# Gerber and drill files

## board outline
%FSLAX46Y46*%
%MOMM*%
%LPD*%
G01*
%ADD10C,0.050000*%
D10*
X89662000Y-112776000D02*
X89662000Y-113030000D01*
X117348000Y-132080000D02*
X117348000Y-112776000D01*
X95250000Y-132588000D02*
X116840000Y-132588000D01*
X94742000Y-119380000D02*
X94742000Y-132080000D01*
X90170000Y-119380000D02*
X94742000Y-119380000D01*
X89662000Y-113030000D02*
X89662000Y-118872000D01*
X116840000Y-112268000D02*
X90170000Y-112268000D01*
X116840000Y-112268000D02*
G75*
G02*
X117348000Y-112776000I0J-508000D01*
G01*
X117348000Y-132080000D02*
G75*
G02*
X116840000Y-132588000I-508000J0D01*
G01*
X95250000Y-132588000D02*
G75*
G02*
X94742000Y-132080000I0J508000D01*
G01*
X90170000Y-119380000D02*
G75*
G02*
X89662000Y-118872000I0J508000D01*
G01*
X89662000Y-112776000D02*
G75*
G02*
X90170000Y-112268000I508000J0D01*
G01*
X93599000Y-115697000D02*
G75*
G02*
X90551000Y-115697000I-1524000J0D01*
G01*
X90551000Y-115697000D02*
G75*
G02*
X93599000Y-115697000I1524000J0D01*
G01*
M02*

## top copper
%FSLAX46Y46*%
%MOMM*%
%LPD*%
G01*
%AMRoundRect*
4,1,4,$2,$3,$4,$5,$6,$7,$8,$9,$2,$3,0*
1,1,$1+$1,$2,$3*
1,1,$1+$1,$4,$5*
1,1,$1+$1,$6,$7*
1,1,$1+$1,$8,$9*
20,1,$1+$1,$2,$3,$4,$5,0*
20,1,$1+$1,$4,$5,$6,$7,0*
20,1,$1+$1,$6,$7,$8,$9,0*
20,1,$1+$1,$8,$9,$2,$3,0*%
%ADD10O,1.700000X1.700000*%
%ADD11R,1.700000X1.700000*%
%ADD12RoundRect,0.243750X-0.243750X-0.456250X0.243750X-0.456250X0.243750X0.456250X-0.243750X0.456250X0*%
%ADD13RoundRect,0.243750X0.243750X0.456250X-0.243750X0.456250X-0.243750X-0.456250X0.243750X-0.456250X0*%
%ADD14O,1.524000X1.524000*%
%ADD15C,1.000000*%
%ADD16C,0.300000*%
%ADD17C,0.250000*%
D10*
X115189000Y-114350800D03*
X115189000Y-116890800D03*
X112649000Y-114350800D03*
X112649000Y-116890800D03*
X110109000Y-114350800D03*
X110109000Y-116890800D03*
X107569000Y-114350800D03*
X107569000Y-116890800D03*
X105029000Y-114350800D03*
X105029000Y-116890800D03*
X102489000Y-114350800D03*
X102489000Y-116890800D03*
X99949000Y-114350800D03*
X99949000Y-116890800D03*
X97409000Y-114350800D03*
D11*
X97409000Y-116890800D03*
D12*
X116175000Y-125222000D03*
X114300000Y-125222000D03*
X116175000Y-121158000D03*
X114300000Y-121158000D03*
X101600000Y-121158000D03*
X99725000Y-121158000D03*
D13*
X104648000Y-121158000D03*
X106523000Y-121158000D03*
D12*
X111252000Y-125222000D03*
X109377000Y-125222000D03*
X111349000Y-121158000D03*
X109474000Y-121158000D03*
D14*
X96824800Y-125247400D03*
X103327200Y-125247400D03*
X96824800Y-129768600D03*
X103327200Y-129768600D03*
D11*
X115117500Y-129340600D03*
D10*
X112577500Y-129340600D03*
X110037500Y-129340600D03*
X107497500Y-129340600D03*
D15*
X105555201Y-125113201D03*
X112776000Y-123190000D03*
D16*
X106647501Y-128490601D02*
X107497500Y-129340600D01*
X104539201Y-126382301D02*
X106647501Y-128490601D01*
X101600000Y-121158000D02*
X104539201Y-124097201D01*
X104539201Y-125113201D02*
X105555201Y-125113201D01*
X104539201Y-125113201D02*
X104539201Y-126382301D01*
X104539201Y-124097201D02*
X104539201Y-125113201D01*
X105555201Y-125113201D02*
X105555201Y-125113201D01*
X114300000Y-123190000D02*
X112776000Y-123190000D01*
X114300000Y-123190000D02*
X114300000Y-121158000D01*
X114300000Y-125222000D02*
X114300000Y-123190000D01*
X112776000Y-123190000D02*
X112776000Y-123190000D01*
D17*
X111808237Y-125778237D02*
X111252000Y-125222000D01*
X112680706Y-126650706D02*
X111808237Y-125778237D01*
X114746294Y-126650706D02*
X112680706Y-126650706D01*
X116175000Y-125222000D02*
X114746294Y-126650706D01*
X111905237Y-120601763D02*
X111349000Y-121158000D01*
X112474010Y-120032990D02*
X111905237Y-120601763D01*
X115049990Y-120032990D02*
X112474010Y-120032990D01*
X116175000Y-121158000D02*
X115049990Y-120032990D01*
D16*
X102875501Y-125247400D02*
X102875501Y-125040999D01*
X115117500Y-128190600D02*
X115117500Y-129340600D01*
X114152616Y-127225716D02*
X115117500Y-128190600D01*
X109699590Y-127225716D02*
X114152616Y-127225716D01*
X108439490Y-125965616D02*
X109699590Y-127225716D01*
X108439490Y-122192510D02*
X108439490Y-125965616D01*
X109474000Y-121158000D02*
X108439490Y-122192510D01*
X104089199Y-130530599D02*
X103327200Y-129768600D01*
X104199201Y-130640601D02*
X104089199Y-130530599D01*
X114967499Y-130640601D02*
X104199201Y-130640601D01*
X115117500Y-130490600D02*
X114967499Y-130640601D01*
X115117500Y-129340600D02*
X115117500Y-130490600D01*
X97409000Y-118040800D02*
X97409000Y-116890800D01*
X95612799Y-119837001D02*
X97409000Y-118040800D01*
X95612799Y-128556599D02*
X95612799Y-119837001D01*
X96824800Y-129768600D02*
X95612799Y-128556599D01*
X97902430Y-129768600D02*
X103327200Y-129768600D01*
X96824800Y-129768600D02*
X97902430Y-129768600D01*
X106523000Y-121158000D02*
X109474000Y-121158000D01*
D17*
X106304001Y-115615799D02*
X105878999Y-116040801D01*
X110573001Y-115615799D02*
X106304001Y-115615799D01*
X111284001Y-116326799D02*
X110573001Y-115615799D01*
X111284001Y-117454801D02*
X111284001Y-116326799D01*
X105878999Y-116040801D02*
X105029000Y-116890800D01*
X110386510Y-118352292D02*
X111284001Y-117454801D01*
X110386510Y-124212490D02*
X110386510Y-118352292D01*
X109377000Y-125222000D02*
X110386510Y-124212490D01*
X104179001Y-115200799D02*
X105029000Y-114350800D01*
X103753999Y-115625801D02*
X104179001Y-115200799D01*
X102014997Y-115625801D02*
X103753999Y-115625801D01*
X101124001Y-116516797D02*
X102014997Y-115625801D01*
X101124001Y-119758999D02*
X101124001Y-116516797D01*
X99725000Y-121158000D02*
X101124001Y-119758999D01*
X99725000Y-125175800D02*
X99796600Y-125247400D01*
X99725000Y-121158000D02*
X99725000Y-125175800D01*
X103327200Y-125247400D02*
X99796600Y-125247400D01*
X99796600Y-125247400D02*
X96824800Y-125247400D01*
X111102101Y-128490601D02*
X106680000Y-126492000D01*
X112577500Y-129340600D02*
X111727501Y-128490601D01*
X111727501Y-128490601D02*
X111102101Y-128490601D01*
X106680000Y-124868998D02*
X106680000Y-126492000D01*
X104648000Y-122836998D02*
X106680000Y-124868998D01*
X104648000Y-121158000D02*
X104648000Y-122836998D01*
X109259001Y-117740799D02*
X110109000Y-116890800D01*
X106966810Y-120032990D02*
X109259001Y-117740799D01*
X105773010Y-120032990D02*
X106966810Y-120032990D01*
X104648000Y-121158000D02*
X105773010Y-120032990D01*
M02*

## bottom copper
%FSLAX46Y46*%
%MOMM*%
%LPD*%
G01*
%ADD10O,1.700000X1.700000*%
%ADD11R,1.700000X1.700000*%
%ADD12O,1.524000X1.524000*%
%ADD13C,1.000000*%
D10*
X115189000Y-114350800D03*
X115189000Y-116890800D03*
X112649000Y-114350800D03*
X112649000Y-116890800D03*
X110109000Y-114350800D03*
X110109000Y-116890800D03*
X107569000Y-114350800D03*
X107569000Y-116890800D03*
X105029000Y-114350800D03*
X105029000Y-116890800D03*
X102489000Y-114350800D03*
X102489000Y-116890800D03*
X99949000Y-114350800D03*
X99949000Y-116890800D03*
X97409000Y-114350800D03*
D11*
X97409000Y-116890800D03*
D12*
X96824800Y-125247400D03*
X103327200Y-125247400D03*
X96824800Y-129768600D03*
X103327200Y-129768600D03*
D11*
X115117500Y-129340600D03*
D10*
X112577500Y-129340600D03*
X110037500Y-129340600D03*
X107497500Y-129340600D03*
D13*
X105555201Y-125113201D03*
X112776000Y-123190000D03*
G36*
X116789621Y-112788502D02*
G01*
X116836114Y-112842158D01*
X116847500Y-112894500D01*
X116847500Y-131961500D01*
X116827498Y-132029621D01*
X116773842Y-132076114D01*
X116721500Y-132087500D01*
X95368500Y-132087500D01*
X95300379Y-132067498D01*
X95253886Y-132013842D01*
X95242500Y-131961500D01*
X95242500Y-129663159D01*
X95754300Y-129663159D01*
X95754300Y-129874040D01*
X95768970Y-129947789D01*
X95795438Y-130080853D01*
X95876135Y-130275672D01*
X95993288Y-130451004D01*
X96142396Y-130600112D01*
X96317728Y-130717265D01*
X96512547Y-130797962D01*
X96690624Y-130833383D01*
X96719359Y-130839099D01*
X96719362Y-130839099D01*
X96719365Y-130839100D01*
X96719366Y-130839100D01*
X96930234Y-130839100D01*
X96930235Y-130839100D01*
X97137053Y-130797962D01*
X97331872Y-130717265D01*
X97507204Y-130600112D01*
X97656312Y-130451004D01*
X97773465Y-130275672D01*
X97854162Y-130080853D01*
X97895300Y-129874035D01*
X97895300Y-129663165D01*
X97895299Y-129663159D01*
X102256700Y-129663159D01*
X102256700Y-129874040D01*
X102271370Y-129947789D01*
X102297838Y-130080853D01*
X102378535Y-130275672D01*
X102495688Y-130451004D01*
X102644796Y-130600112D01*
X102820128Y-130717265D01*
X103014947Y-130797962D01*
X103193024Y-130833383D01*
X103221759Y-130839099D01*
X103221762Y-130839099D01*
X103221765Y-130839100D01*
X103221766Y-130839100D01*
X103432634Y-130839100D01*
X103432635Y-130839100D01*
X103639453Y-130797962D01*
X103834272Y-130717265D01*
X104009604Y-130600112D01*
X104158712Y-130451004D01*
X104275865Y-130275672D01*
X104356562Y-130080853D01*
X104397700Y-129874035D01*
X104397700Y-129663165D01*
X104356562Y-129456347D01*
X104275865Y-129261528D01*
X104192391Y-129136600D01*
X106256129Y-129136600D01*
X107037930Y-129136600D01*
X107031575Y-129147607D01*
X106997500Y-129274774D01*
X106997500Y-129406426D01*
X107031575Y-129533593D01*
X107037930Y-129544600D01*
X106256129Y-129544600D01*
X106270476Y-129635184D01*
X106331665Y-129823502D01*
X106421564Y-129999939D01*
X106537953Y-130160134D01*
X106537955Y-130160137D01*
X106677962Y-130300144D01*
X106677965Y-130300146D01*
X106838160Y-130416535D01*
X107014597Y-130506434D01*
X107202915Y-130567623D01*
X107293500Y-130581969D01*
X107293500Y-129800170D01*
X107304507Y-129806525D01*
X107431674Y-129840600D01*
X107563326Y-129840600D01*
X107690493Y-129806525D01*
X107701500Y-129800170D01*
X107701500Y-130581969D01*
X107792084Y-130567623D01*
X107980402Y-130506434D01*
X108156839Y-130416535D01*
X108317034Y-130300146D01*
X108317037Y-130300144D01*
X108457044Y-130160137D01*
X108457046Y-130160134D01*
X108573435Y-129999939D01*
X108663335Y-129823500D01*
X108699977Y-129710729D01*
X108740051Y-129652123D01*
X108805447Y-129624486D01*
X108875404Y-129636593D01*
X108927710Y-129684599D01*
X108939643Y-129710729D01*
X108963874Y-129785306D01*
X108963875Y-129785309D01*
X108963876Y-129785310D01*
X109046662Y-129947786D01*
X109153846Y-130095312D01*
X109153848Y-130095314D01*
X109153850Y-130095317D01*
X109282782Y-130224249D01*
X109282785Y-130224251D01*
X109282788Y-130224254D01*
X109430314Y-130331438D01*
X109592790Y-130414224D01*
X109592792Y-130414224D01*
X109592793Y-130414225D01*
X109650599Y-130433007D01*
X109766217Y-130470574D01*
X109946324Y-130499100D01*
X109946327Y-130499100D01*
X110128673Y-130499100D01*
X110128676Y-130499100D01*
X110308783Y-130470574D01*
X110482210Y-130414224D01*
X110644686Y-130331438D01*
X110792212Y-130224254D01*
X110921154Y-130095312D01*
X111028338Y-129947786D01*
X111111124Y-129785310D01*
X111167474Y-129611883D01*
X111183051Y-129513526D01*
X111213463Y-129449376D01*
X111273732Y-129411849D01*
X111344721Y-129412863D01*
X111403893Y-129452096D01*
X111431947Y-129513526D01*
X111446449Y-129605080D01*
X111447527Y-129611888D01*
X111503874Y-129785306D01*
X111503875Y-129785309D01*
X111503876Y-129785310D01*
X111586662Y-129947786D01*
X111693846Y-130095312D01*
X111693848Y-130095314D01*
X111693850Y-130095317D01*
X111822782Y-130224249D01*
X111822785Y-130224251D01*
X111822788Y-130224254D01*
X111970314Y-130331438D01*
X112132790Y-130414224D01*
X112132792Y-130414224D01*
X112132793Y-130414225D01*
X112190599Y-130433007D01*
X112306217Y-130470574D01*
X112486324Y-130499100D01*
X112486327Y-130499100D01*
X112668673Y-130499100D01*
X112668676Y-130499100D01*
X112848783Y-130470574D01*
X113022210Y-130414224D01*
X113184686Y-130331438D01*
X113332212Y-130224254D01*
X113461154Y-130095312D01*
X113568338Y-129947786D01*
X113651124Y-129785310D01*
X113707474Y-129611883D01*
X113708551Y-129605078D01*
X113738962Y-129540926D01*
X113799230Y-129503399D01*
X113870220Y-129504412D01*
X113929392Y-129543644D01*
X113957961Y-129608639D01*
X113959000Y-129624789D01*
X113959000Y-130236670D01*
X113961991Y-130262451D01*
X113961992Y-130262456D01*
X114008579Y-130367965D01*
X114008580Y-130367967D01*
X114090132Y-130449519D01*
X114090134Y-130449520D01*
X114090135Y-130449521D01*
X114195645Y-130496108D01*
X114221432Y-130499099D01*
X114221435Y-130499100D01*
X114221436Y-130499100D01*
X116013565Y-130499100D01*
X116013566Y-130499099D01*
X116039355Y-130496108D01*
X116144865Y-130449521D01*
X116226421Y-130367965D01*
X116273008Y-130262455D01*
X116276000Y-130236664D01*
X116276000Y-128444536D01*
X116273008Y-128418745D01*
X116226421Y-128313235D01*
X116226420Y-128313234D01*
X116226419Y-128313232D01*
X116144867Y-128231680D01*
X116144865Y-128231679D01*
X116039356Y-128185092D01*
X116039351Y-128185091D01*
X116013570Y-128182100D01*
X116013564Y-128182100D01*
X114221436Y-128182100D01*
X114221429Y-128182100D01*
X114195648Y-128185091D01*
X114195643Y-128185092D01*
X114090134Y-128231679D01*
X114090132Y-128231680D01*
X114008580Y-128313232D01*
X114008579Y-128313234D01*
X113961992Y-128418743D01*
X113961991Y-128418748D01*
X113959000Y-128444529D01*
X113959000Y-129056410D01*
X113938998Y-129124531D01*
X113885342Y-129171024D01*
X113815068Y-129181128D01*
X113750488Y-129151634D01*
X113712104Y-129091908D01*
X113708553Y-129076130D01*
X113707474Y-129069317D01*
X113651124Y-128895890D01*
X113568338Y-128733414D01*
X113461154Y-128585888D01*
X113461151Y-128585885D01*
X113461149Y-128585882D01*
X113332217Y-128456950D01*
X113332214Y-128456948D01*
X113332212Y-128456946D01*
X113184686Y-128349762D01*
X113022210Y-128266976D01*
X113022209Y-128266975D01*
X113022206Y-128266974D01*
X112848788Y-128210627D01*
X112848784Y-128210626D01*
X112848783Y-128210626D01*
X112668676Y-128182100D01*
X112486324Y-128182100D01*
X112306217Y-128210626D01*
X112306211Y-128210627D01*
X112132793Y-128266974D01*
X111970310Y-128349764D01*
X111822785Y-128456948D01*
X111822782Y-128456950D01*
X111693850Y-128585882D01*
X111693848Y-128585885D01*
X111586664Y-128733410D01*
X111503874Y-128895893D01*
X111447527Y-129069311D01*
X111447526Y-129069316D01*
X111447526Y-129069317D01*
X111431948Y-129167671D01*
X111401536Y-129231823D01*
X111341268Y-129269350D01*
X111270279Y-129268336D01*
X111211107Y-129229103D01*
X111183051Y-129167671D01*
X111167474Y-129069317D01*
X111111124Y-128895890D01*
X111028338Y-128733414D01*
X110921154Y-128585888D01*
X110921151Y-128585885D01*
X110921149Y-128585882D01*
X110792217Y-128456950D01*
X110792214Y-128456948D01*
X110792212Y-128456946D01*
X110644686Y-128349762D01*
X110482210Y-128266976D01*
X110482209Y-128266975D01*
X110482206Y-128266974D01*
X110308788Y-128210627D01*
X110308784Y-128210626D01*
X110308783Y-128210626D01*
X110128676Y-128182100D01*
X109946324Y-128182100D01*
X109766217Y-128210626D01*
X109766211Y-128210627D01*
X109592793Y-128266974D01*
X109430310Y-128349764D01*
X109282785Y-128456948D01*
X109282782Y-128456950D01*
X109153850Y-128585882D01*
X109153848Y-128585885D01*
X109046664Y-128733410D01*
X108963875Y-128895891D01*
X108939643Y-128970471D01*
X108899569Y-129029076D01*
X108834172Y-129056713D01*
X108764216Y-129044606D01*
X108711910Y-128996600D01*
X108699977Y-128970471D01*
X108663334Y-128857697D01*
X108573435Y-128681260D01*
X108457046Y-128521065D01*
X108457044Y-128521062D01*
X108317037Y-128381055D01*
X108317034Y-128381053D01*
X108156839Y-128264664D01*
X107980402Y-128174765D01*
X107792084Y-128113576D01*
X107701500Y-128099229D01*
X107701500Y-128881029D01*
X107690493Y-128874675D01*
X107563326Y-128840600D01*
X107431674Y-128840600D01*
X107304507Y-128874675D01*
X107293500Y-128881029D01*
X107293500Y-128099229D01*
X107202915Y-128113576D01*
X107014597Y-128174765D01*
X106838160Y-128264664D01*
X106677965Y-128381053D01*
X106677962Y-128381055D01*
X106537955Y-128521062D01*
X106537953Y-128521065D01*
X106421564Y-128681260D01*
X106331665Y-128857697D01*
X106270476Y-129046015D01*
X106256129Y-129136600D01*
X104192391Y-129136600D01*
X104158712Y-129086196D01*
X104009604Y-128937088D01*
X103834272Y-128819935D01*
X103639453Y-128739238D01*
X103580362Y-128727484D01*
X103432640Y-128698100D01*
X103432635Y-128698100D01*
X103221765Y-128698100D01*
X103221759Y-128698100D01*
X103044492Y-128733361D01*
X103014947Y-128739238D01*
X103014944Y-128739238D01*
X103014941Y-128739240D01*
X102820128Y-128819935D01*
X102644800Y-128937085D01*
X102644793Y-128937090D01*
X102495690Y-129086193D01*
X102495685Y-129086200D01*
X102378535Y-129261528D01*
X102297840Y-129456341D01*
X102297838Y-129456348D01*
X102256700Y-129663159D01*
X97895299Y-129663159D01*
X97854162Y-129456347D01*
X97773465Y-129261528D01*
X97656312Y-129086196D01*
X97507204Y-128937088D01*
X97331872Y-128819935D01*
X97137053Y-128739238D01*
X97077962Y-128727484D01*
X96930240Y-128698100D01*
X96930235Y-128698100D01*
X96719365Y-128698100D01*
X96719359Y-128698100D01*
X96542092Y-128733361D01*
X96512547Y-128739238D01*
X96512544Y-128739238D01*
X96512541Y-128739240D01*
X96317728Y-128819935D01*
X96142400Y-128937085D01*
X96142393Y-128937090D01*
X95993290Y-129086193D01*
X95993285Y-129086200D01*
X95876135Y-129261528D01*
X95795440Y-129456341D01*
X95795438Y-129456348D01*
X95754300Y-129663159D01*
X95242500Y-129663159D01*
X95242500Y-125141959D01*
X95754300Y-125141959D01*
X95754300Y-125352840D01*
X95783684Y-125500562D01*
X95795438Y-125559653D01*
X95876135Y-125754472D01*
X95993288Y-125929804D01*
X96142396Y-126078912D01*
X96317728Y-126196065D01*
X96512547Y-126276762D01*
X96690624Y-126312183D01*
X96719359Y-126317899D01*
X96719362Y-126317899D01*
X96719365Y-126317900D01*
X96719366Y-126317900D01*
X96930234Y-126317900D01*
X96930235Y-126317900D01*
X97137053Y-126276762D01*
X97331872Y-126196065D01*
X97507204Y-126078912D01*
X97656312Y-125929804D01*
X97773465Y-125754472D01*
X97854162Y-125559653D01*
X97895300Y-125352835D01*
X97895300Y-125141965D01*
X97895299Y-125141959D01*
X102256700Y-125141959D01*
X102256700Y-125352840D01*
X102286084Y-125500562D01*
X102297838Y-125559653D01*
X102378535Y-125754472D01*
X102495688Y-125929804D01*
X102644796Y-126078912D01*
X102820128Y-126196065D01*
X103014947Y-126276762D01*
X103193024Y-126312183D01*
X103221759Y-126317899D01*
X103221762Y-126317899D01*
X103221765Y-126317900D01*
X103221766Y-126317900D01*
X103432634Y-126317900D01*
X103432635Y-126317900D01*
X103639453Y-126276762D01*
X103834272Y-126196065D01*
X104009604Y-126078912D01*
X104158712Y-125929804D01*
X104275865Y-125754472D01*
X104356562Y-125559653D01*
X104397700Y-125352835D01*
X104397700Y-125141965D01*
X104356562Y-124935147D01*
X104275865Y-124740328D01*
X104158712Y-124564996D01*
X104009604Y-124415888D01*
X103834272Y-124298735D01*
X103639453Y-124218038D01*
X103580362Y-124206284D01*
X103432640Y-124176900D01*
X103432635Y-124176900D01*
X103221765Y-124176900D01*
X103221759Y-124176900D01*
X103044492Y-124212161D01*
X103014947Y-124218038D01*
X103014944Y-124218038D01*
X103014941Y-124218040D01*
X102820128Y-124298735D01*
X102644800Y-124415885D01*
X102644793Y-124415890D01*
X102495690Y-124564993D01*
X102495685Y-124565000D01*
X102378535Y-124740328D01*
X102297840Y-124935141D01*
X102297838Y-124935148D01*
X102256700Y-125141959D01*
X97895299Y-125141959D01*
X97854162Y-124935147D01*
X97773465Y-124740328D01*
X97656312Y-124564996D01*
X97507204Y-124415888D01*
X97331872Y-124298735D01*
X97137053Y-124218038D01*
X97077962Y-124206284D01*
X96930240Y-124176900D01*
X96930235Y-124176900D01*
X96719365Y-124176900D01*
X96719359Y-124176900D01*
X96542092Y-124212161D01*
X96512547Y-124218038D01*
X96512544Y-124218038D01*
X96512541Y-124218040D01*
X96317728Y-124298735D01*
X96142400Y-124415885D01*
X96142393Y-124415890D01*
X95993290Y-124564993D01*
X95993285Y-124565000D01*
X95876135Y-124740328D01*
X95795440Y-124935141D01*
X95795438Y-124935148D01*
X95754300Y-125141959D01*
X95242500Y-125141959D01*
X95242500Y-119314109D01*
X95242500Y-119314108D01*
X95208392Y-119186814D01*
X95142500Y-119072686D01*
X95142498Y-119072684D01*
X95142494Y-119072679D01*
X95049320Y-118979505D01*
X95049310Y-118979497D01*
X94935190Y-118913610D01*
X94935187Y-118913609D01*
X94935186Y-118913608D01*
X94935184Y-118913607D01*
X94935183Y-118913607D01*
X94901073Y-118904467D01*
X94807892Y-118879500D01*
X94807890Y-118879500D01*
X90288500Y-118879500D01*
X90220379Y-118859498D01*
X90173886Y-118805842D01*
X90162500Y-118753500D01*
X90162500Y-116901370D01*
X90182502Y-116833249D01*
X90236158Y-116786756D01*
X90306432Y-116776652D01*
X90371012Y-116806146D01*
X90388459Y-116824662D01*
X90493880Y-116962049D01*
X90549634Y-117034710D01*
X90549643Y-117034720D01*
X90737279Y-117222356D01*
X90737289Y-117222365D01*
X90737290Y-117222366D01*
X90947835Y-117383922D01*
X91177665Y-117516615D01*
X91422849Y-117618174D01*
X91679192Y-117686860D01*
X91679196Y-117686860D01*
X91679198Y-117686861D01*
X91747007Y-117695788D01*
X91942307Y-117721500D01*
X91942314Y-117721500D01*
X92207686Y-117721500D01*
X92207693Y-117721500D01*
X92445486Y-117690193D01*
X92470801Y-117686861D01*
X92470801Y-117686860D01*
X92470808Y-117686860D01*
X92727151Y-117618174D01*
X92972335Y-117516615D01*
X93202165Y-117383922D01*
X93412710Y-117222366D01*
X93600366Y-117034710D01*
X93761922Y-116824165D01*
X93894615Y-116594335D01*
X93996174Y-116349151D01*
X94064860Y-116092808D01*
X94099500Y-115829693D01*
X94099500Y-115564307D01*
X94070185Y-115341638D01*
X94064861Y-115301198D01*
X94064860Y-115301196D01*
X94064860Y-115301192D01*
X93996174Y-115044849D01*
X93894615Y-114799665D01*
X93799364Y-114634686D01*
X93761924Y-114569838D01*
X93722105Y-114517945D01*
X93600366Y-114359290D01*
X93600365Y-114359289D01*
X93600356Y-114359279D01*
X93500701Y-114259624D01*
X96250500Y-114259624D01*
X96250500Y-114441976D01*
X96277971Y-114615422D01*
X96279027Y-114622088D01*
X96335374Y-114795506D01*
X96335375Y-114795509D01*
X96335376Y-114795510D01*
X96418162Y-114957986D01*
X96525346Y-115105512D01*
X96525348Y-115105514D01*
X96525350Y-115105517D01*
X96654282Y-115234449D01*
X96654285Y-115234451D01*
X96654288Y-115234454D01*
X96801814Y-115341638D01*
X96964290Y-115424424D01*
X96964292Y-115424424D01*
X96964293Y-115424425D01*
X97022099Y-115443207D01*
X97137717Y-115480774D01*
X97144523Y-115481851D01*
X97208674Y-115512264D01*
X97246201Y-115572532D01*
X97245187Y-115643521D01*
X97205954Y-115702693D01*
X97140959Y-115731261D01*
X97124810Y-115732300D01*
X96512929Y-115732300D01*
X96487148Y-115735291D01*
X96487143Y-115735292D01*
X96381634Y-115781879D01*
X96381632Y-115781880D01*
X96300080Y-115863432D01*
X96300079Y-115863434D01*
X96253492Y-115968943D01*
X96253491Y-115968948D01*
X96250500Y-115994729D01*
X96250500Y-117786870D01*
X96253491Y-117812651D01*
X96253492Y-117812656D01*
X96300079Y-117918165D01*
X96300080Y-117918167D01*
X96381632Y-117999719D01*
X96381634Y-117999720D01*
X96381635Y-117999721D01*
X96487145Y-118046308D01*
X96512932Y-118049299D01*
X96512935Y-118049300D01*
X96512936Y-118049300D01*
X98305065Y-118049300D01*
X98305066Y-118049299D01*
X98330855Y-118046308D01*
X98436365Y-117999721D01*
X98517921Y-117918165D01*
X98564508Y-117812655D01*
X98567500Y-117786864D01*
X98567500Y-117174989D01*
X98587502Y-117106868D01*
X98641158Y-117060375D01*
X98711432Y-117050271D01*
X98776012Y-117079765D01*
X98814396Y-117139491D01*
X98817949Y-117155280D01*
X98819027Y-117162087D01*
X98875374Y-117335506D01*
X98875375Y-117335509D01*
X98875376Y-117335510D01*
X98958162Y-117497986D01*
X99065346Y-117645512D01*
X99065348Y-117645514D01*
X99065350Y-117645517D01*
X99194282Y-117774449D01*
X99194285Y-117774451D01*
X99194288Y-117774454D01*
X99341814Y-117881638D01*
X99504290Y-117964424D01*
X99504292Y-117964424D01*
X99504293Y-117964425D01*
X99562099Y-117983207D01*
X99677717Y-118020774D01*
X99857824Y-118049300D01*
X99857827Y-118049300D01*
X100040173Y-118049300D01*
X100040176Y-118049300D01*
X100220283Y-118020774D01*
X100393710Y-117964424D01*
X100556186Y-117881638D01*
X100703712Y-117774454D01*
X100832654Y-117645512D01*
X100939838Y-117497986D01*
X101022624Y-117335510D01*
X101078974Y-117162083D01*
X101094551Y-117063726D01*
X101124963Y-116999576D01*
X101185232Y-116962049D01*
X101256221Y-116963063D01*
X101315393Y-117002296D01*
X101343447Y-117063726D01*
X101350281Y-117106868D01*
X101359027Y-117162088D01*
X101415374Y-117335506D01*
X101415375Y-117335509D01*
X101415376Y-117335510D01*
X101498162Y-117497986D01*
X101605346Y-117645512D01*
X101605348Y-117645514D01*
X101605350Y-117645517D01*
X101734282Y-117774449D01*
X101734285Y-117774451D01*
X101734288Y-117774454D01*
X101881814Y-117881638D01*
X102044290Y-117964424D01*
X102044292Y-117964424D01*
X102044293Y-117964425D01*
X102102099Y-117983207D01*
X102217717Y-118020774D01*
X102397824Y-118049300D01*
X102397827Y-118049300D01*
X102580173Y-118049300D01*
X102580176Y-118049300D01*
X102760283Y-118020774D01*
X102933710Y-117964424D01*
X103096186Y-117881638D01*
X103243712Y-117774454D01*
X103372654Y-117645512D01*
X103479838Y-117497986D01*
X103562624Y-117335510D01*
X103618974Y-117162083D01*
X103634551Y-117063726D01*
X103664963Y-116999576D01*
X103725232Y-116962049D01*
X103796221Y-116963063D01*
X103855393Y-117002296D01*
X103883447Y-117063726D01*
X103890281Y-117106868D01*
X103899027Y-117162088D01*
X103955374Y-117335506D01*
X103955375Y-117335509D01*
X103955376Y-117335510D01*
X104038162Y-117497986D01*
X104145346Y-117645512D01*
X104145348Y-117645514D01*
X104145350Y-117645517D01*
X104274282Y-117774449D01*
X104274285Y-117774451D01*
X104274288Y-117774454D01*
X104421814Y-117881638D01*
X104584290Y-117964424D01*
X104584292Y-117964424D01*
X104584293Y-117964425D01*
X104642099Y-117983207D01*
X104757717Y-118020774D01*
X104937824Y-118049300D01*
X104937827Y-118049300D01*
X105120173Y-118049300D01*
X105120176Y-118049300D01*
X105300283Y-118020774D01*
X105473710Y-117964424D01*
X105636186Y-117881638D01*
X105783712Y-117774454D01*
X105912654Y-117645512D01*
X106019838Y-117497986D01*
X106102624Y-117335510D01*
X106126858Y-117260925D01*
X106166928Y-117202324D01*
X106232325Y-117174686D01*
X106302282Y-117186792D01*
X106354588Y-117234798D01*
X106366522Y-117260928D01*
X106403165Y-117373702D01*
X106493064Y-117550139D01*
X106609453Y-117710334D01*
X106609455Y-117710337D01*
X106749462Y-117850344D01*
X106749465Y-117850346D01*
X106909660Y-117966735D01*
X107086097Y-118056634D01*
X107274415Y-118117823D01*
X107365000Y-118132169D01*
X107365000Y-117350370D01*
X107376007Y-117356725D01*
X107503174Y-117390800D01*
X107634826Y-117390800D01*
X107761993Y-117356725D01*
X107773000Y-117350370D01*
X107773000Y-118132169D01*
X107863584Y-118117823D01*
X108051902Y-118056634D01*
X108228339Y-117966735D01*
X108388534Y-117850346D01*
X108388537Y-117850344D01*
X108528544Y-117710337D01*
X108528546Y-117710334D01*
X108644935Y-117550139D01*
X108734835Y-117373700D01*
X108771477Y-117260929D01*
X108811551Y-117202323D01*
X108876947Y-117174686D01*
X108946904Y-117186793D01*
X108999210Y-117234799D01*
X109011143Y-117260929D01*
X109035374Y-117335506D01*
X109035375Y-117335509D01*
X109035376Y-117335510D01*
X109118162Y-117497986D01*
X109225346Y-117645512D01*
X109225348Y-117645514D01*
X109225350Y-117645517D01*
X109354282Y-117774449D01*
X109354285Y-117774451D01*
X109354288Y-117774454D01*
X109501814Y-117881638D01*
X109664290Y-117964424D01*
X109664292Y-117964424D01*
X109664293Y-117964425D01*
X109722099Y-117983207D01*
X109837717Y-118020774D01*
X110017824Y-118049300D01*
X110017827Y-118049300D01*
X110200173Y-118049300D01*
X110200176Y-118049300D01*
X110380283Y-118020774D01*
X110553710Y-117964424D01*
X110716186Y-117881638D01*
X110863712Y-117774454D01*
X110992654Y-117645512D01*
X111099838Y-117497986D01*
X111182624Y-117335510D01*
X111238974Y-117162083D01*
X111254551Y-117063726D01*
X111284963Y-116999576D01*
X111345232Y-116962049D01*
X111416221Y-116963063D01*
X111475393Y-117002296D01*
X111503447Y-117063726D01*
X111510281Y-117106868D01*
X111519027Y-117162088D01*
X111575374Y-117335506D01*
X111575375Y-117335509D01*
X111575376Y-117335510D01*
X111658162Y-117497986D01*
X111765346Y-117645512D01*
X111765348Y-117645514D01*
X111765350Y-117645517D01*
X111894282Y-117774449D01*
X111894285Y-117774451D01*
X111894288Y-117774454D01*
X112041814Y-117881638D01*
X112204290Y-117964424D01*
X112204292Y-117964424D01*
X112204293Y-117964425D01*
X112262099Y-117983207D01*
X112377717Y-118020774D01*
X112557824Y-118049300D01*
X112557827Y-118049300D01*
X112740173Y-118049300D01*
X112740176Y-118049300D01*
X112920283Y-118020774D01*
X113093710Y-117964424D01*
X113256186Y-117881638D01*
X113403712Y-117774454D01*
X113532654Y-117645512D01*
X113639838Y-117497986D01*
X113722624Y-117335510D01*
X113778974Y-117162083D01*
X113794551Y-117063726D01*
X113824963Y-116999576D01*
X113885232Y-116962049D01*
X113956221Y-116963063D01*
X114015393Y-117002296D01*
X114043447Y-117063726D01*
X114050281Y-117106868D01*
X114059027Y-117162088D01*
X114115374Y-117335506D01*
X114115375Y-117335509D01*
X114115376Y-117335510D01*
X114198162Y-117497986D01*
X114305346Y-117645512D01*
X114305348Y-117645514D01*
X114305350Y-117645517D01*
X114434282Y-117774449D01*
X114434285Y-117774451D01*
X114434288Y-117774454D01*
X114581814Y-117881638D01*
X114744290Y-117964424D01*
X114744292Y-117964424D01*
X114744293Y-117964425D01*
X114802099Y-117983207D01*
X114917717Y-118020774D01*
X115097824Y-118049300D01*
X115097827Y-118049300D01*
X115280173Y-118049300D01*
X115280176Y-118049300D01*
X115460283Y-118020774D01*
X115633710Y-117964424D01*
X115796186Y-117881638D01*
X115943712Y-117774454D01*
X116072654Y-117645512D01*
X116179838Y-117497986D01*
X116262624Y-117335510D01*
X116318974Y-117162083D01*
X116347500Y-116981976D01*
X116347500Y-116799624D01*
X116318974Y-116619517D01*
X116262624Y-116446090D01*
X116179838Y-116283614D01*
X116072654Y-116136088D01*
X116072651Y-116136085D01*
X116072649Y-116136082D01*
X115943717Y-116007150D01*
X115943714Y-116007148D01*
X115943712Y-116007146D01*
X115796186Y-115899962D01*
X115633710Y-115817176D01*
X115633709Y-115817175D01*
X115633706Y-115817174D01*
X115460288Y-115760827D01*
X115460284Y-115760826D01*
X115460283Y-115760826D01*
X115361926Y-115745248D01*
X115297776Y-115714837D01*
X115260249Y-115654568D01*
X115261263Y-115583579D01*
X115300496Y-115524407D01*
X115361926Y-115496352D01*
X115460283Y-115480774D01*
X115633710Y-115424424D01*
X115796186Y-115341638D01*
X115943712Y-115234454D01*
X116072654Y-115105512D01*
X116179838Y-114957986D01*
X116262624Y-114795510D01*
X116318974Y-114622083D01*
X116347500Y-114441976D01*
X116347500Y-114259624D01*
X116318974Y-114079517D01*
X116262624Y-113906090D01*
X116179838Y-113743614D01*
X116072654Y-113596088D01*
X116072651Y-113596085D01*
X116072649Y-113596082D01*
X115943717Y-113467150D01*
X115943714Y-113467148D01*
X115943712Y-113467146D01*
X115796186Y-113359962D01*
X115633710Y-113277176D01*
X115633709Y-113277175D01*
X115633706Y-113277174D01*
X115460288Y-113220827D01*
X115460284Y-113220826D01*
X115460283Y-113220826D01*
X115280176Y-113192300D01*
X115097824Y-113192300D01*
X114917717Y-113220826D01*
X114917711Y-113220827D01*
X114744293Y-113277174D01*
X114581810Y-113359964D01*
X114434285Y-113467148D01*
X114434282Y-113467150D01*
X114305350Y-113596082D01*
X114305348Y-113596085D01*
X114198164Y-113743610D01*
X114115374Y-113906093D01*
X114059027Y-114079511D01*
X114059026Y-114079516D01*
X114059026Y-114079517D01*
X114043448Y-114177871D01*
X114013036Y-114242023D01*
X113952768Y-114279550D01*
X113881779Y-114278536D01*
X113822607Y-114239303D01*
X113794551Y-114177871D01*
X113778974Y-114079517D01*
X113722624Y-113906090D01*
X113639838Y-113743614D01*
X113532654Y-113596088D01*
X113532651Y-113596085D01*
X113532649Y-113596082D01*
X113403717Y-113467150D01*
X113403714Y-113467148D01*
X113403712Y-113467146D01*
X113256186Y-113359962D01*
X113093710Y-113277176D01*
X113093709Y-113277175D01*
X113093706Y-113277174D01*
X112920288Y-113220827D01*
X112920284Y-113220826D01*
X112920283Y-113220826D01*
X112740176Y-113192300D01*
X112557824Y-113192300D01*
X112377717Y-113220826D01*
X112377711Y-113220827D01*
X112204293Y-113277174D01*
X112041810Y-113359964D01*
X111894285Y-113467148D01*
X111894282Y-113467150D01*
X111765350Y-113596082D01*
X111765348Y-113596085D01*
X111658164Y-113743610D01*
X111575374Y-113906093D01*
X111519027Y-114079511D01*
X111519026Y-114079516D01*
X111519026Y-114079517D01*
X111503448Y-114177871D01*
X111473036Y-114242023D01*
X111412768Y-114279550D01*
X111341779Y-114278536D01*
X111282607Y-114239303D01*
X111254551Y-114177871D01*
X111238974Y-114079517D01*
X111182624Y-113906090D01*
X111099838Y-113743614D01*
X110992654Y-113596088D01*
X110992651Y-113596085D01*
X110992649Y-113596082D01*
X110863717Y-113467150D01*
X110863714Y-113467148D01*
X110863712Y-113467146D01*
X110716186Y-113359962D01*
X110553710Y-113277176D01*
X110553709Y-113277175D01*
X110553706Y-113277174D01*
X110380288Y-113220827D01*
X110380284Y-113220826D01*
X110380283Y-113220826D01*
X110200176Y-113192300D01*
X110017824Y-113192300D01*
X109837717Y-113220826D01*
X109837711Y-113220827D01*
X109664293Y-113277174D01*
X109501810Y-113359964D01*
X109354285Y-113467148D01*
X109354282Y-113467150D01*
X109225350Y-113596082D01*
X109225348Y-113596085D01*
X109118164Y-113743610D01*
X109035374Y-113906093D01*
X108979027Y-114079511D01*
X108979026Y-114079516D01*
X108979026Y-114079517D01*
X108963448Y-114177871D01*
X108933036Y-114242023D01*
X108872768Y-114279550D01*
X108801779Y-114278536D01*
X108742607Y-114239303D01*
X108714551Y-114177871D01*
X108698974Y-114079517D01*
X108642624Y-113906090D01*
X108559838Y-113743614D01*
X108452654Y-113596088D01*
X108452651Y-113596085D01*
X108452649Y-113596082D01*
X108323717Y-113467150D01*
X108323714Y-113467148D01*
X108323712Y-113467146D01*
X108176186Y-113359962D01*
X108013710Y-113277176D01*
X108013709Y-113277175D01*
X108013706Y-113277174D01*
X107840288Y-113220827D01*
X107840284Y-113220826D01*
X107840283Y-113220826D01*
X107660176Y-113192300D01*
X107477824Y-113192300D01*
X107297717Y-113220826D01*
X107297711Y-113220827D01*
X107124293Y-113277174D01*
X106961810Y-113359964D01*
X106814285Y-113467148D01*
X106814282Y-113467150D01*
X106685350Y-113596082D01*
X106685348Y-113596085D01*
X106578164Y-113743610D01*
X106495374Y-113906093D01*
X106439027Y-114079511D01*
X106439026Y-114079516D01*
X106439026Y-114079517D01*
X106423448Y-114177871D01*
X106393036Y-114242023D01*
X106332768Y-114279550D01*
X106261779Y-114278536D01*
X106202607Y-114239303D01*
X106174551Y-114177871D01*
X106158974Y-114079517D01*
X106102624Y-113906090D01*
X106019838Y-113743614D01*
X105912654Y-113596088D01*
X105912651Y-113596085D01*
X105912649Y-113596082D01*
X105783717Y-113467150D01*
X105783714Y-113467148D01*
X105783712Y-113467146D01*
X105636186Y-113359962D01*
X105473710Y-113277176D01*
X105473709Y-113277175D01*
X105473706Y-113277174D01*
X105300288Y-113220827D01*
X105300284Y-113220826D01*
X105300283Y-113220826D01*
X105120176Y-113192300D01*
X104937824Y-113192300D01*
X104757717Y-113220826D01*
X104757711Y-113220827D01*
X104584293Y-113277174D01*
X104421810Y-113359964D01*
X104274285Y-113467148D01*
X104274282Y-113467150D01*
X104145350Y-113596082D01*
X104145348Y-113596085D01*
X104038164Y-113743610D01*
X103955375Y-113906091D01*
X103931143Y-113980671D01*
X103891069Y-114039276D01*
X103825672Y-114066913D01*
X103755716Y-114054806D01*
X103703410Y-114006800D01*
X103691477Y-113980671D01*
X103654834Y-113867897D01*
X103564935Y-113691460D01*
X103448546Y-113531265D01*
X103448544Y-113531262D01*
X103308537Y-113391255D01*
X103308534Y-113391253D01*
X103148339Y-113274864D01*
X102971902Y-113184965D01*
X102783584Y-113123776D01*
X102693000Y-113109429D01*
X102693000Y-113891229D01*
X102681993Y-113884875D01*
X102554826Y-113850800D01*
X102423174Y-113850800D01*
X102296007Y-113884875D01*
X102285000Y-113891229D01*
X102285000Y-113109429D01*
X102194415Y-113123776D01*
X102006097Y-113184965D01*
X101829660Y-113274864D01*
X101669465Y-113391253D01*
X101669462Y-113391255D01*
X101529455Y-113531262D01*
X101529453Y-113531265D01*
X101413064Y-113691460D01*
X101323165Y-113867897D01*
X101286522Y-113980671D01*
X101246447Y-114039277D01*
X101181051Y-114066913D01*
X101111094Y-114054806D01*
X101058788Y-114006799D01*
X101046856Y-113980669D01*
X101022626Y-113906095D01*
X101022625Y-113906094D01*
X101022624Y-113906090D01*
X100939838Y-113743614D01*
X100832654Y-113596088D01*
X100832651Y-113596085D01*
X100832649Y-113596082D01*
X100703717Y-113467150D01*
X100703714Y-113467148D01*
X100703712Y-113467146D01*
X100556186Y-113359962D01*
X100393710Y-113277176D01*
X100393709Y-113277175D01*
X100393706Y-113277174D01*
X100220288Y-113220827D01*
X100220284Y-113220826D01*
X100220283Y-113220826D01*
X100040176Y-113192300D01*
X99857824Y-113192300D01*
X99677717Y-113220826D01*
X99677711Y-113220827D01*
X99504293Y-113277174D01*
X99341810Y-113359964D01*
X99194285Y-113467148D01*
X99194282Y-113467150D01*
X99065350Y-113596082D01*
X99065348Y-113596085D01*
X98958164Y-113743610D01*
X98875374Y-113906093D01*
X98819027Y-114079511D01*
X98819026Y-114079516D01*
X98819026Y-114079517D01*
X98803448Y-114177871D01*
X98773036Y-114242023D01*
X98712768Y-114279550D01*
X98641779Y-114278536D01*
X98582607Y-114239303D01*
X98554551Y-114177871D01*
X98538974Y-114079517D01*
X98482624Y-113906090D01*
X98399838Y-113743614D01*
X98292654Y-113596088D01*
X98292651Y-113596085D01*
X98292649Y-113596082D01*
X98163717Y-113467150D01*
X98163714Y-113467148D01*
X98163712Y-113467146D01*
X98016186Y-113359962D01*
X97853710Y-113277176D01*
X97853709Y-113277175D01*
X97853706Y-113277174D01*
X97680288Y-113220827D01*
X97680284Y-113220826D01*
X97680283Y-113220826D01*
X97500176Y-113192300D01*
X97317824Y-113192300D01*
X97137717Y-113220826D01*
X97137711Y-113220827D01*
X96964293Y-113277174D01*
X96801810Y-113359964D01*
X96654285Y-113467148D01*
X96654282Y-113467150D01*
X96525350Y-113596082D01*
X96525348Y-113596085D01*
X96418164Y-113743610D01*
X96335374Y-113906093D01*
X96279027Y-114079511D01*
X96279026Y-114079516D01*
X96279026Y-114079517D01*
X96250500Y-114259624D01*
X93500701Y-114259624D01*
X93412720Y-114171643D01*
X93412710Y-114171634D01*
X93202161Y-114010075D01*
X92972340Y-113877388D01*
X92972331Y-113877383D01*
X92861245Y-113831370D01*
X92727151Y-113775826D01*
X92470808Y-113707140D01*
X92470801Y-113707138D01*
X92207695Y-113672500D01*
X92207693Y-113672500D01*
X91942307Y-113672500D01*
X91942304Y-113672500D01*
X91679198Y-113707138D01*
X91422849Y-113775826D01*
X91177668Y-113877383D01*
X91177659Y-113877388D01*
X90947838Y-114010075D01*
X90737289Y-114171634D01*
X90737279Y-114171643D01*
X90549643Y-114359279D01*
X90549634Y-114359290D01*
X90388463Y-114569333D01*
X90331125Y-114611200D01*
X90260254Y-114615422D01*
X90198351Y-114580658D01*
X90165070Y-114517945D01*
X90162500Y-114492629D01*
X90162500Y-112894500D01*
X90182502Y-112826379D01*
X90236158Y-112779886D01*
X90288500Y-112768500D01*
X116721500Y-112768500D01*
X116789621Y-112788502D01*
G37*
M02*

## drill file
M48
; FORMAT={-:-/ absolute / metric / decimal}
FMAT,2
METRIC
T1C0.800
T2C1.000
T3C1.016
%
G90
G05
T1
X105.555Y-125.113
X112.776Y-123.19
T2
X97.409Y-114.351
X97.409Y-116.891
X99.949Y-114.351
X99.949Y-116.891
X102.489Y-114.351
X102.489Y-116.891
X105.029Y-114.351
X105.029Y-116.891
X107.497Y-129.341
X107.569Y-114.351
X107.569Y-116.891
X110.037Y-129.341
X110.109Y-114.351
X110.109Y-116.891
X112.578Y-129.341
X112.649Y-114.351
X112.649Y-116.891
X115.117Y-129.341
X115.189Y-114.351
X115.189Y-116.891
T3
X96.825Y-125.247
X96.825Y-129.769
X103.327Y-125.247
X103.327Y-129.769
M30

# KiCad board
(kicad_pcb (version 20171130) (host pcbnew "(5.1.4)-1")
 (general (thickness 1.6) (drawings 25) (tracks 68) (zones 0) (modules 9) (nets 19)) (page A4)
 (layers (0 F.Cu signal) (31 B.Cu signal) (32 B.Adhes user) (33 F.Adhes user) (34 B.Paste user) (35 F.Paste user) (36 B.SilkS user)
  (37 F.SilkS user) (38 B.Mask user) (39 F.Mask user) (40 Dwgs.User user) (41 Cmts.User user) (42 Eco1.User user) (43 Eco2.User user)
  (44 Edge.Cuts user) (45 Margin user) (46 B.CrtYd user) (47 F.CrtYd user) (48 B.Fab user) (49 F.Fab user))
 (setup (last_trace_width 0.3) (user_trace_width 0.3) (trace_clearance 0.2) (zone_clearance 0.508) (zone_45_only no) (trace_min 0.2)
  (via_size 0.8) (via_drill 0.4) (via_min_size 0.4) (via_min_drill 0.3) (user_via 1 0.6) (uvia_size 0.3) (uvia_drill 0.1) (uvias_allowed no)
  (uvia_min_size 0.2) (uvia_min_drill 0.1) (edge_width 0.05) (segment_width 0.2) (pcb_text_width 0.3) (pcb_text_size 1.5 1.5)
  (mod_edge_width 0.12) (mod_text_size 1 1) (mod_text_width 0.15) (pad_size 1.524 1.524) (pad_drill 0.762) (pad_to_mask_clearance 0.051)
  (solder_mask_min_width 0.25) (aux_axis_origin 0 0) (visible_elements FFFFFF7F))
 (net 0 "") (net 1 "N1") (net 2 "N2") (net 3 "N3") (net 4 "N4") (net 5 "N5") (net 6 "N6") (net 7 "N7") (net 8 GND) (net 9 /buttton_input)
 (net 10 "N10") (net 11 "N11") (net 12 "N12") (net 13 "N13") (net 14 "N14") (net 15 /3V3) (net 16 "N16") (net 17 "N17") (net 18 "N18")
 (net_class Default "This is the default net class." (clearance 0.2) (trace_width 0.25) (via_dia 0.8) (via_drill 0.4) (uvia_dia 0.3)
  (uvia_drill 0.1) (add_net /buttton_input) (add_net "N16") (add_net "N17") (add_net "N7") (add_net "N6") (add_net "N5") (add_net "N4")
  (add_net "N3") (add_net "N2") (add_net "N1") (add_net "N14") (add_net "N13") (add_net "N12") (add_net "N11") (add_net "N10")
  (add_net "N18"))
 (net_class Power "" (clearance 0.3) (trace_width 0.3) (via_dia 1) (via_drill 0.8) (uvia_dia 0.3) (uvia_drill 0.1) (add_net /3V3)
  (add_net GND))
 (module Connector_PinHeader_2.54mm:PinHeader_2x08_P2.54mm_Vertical (layer F.Cu) (at 97.409 116.8908 90)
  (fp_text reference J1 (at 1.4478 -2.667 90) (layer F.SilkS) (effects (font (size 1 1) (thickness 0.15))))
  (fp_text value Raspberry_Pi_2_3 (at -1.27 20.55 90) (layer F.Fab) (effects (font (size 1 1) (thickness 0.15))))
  (pad 16 thru_hole oval (at 2.54 17.78 90) (size 1.7 1.7) (drill 1) (layers *.Cu *.Mask) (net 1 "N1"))
  (pad 15 thru_hole oval (at 0 17.78 90) (size 1.7 1.7) (drill 1) (layers *.Cu *.Mask) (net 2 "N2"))
  (pad 14 thru_hole oval (at 2.54 15.24 90) (size 1.7 1.7) (drill 1) (layers *.Cu *.Mask) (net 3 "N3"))
  (pad 13 thru_hole oval (at 0 15.24 90) (size 1.7 1.7) (drill 1) (layers *.Cu *.Mask) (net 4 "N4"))
  (pad 12 thru_hole oval (at 2.54 12.7 90) (size 1.7 1.7) (drill 1) (layers *.Cu *.Mask) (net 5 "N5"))
  (pad 11 thru_hole oval (at 0 12.7 90) (size 1.7 1.7) (drill 1) (layers *.Cu *.Mask) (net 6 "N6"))
  (pad 10 thru_hole oval (at 2.54 10.16 90) (size 1.7 1.7) (drill 1) (layers *.Cu *.Mask) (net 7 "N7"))
  (pad 9 thru_hole oval (at 0 10.16 90) (size 1.7 1.7) (drill 1) (layers *.Cu *.Mask) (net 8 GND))
  (pad 8 thru_hole oval (at 2.54 7.62 90) (size 1.7 1.7) (drill 1) (layers *.Cu *.Mask) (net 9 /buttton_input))
  (pad 7 thru_hole oval (at 0 7.62 90) (size 1.7 1.7) (drill 1) (layers *.Cu *.Mask) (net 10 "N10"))
  (pad 6 thru_hole oval (at 2.54 5.08 90) (size 1.7 1.7) (drill 1) (layers *.Cu *.Mask) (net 8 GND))
  (pad 5 thru_hole oval (at 0 5.08 90) (size 1.7 1.7) (drill 1) (layers *.Cu *.Mask) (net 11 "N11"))
  (pad 4 thru_hole oval (at 2.54 2.54 90) (size 1.7 1.7) (drill 1) (layers *.Cu *.Mask) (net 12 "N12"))
  (pad 3 thru_hole oval (at 0 2.54 90) (size 1.7 1.7) (drill 1) (layers *.Cu *.Mask) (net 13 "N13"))
  (pad 2 thru_hole oval (at 2.54 0 90) (size 1.7 1.7) (drill 1) (layers *.Cu *.Mask) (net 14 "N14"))
  (pad 1 thru_hole rect (at 0 0 90) (size 1.7 1.7) (drill 1) (layers *.Cu *.Mask) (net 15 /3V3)))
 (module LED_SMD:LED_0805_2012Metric (layer F.Cu) (at 115.2375 125.222)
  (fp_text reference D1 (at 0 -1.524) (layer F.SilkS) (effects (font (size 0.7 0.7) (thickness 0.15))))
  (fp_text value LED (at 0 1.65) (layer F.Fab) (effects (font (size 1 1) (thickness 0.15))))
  (pad 2 smd roundrect (at 0.9375 0) (size 0.975 1.4) (layers F.Cu F.Paste F.Mask) (roundrect_rratio 0.25) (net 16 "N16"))
  (pad 1 smd roundrect (at -0.9375 0) (size 0.975 1.4) (layers F.Cu F.Paste F.Mask) (roundrect_rratio 0.25) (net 8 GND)))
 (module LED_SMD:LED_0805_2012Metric (layer F.Cu) (at 115.2375 121.158)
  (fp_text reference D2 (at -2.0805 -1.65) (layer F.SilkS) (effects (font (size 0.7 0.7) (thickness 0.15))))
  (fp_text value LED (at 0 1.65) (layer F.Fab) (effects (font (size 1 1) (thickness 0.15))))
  (pad 2 smd roundrect (at 0.9375 0) (size 0.975 1.4) (layers F.Cu F.Paste F.Mask) (roundrect_rratio 0.25) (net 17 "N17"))
  (pad 1 smd roundrect (at -0.9375 0) (size 0.975 1.4) (layers F.Cu F.Paste F.Mask) (roundrect_rratio 0.25) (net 8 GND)))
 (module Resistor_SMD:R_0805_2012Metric (layer F.Cu) (at 100.6625 121.158)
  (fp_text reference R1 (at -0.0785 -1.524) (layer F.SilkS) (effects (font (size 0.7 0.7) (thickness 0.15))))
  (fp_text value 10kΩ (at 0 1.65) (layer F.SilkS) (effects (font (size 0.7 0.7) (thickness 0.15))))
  (pad 2 smd roundrect (at 0.9375 0) (size 0.975 1.4) (layers F.Cu F.Paste F.Mask) (roundrect_rratio 0.25) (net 8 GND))
  (pad 1 smd roundrect (at -0.9375 0) (size 0.975 1.4) (layers F.Cu F.Paste F.Mask) (roundrect_rratio 0.25) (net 9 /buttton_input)))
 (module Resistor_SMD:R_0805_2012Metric (layer F.Cu) (at 105.5855 121.158 180)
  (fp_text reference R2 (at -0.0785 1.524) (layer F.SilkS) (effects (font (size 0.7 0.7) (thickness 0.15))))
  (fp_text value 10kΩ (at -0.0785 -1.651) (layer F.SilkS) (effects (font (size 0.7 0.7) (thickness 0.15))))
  (pad 2 smd roundrect (at 0.9375 0 180) (size 0.975 1.4) (layers F.Cu F.Paste F.Mask) (roundrect_rratio 0.25) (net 6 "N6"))
  (pad 1 smd roundrect (at -0.9375 0 180) (size 0.975 1.4) (layers F.Cu F.Paste F.Mask) (roundrect_rratio 0.25) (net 15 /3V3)))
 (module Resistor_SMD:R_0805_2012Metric (layer F.Cu) (at 110.3145 125.222)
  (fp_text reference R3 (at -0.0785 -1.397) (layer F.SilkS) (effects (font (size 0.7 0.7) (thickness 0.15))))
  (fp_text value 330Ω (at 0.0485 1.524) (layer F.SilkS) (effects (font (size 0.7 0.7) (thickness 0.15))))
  (pad 2 smd roundrect (at 0.9375 0) (size 0.975 1.4) (layers F.Cu F.Paste F.Mask) (roundrect_rratio 0.25) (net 16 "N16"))
  (pad 1 smd roundrect (at -0.9375 0) (size 0.975 1.4) (layers F.Cu F.Paste F.Mask) (roundrect_rratio 0.25) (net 10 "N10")))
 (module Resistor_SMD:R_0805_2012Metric (layer F.Cu) (at 110.4115 121.158)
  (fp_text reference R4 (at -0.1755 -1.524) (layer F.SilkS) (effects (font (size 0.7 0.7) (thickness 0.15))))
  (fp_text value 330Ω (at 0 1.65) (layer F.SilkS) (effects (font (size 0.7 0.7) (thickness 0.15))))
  (pad 2 smd roundrect (at 0.9375 0) (size 0.975 1.4) (layers F.Cu F.Paste F.Mask) (roundrect_rratio 0.25) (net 17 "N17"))
  (pad 1 smd roundrect (at -0.9375 0) (size 0.975 1.4) (layers F.Cu F.Paste F.Mask) (roundrect_rratio 0.25) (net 15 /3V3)))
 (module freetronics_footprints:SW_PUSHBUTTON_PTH (layer F.Cu) (at 100.076 127.508 180)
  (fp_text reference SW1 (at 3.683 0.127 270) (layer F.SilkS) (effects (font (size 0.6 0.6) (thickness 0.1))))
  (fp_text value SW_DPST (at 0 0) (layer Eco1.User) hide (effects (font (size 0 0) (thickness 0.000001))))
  (pad 2 thru_hole oval (at 3.2512 2.2606 180) (size 1.524 1.524) (drill 1.016) (layers *.Cu *.Mask) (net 9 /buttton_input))
  (pad 2 thru_hole oval (at -3.2512 2.2606 180) (size 1.524 1.524) (drill 1.016) (layers *.Cu *.Mask) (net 9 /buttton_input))
  (pad 1 thru_hole oval (at 3.2512 -2.2606 180) (size 1.524 1.524) (drill 1.016) (layers *.Cu *.Mask) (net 15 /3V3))
  (pad 1 thru_hole oval (at -3.2512 -2.2606 180) (size 1.524 1.524) (drill 1.016) (layers *.Cu *.Mask) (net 15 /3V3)))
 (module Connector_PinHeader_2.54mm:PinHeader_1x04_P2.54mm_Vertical (layer F.Cu) (at 115.1175 129.3406 270)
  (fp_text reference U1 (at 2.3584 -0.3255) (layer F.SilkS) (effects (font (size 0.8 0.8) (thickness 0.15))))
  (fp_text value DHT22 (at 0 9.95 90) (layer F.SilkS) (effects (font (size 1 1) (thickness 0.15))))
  (pad 1 thru_hole rect (at 0 0 270) (size 1.7 1.7) (drill 1) (layers *.Cu *.Mask) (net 15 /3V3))
  (pad 2 thru_hole oval (at 0 2.54 270) (size 1.7 1.7) (drill 1) (layers *.Cu *.Mask) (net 6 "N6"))
  (pad 3 thru_hole oval (at 0 5.08 270) (size 1.7 1.7) (drill 1) (layers *.Cu *.Mask) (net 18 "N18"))
  (pad 4 thru_hole oval (at 0 7.62 270) (size 1.7 1.7) (drill 1) (layers *.Cu *.Mask) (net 8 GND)))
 (gr_line (start 89.662 112.776) (end 89.662 113.03) (layer Edge.Cuts) (width 0.05))
 (gr_line (start 117.348 132.08) (end 117.348 112.776) (layer Edge.Cuts) (width 0.05))
 (gr_line (start 95.25 132.588) (end 116.84 132.588) (layer Edge.Cuts) (width 0.05))
 (gr_line (start 94.742 119.38) (end 94.742 132.08) (layer Edge.Cuts) (width 0.05))
 (gr_line (start 90.17 119.38) (end 94.742 119.38) (layer Edge.Cuts) (width 0.05))
 (gr_line (start 89.662 113.03) (end 89.662 118.872) (layer Edge.Cuts) (width 0.05))
 (gr_line (start 116.84 112.268) (end 90.17 112.268) (layer Edge.Cuts) (width 0.05))
 (gr_arc (start 116.84 112.776) (end 117.348 112.776) (angle -90) (layer Edge.Cuts) (width 0.05))
 (gr_arc (start 116.84 132.08) (end 116.84 132.588) (angle -90) (layer Edge.Cuts) (width 0.05))
 (gr_arc (start 95.25 132.08) (end 94.742 132.08) (angle -90) (layer Edge.Cuts) (width 0.05))
 (gr_arc (start 90.17 118.872) (end 89.662 118.872) (angle -90) (layer Edge.Cuts) (width 0.05))
 (gr_arc (start 90.17 112.776) (end 90.17 112.268) (angle -90) (layer Edge.Cuts) (width 0.05))
 (gr_circle (center 92.075 115.697) (end 93.599 115.697) (layer Edge.Cuts) (width 0.05))
 (segment (start 106.647501 128.490601) (end 107.4975 129.3406) (width 0.3) (layer F.Cu) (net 8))
 (segment (start 104.539201 126.382301) (end 106.647501 128.490601) (width 0.3) (layer F.Cu) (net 8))
 (segment (start 101.6 121.158) (end 104.539201 124.097201) (width 0.3) (layer F.Cu) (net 8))
 (segment (start 104.539201 125.113201) (end 105.555201 125.113201) (width 0.3) (layer F.Cu) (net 8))
 (segment (start 104.539201 125.113201) (end 104.539201 126.382301) (width 0.3) (layer F.Cu) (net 8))
 (segment (start 104.539201 124.097201) (end 104.539201 125.113201) (width 0.3) (layer F.Cu) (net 8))
 (segment (start 105.555201 125.113201) (end 105.555201 125.113201) (width 0.3) (layer F.Cu) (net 8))
 (via (at 105.555201 125.113201) (size 1) (drill 0.8) (layers F.Cu B.Cu) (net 8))
 (segment (start 114.3 123.19) (end 112.776 123.19) (width 0.3) (layer F.Cu) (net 8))
 (segment (start 114.3 123.19) (end 114.3 121.158) (width 0.3) (layer F.Cu) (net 8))
 (segment (start 114.3 125.222) (end 114.3 123.19) (width 0.3) (layer F.Cu) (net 8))
 (segment (start 112.776 123.19) (end 112.776 123.19) (width 0.3) (layer F.Cu) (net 8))
 (via (at 112.776 123.19) (size 1) (drill 0.8) (layers F.Cu B.Cu) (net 8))
 (segment (start 111.808237 125.778237) (end 111.252 125.222) (width 0.25) (layer F.Cu) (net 16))
 (segment (start 112.680706 126.650706) (end 111.808237 125.778237) (width 0.25) (layer F.Cu) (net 16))
 (segment (start 114.746294 126.650706) (end 112.680706 126.650706) (width 0.25) (layer F.Cu) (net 16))
 (segment (start 116.175 125.222) (end 114.746294 126.650706) (width 0.25) (layer F.Cu) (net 16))
 (segment (start 111.905237 120.601763) (end 111.349 121.158) (width 0.25) (layer F.Cu) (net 17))
 (segment (start 112.47401 120.03299) (end 111.905237 120.601763) (width 0.25) (layer F.Cu) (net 17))
 (segment (start 115.04999 120.03299) (end 112.47401 120.03299) (width 0.25) (layer F.Cu) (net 17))
 (segment (start 116.175 121.158) (end 115.04999 120.03299) (width 0.25) (layer F.Cu) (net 17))
 (segment (start 102.875501 125.2474) (end 102.875501 125.040999) (width 0.3) (layer F.Cu) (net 9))
 (segment (start 115.1175 128.1906) (end 115.1175 129.3406) (width 0.3) (layer F.Cu) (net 15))
 (segment (start 114.152616 127.225716) (end 115.1175 128.1906) (width 0.3) (layer F.Cu) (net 15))
 (segment (start 109.69959 127.225716) (end 114.152616 127.225716) (width 0.3) (layer F.Cu) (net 15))
 (segment (start 108.43949 125.965616) (end 109.69959 127.225716) (width 0.3) (layer F.Cu) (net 15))
 (segment (start 108.43949 122.19251) (end 108.43949 125.965616) (width 0.3) (layer F.Cu) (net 15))
 (segment (start 109.474 121.158) (end 108.43949 122.19251) (width 0.3) (layer F.Cu) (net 15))
 (segment (start 104.089199 130.530599) (end 103.3272 129.7686) (width 0.3) (layer F.Cu) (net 15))
 (segment (start 104.199201 130.640601) (end 104.089199 130.530599) (width 0.3) (layer F.Cu) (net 15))
 (segment (start 114.967499 130.640601) (end 104.199201 130.640601) (width 0.3) (layer F.Cu) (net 15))
 (segment (start 115.1175 130.4906) (end 114.967499 130.640601) (width 0.3) (layer F.Cu) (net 15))
 (segment (start 115.1175 129.3406) (end 115.1175 130.4906) (width 0.3) (layer F.Cu) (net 15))
 (segment (start 97.409 118.0408) (end 97.409 116.8908) (width 0.3) (layer F.Cu) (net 15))
 (segment (start 95.612799 119.837001) (end 97.409 118.0408) (width 0.3) (layer F.Cu) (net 15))
 (segment (start 95.612799 128.556599) (end 95.612799 119.837001) (width 0.3) (layer F.Cu) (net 15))
 (segment (start 96.8248 129.7686) (end 95.612799 128.556599) (width 0.3) (layer F.Cu) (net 15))
 (segment (start 97.90243 129.7686) (end 103.3272 129.7686) (width 0.3) (layer F.Cu) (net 15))
 (segment (start 96.8248 129.7686) (end 97.90243 129.7686) (width 0.3) (layer F.Cu) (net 15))
 (segment (start 106.523 121.158) (end 109.474 121.158) (width 0.3) (layer F.Cu) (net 15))
 (segment (start 106.304001 115.615799) (end 105.878999 116.040801) (width 0.25) (layer F.Cu) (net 10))
 (segment (start 110.573001 115.615799) (end 106.304001 115.615799) (width 0.25) (layer F.Cu) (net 10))
 (segment (start 111.284001 116.326799) (end 110.573001 115.615799) (width 0.25) (layer F.Cu) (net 10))
 (segment (start 111.284001 117.454801) (end 111.284001 116.326799) (width 0.25) (layer F.Cu) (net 10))
 (segment (start 105.878999 116.040801) (end 105.029 116.8908) (width 0.25) (layer F.Cu) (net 10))
 (segment (start 110.38651 118.352292) (end 111.284001 117.454801) (width 0.25) (layer F.Cu) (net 10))
 (segment (start 110.38651 124.21249) (end 110.38651 118.352292) (width 0.25) (layer F.Cu) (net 10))
 (segment (start 109.377 125.222) (end 110.38651 124.21249) (width 0.25) (layer F.Cu) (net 10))
 (segment (start 104.179001 115.200799) (end 105.029 114.3508) (width 0.25) (layer F.Cu) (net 9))
 (segment (start 103.753999 115.625801) (end 104.179001 115.200799) (width 0.25) (layer F.Cu) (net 9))
 (segment (start 102.014997 115.625801) (end 103.753999 115.625801) (width 0.25) (layer F.Cu) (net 9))
 (segment (start 101.124001 116.516797) (end 102.014997 115.625801) (width 0.25) (layer F.Cu) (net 9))
 (segment (start 101.124001 119.758999) (end 101.124001 116.516797) (width 0.25) (layer F.Cu) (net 9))
 (segment (start 99.725 121.158) (end 101.124001 119.758999) (width 0.25) (layer F.Cu) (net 9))
 (segment (start 99.725 125.1758) (end 99.7966 125.2474) (width 0.25) (layer F.Cu) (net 9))
 (segment (start 99.725 121.158) (end 99.725 125.1758) (width 0.25) (layer F.Cu) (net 9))
 (segment (start 103.3272 125.2474) (end 99.7966 125.2474) (width 0.25) (layer F.Cu) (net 9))
 (segment (start 99.7966 125.2474) (end 96.8248 125.2474) (width 0.25) (layer F.Cu) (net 9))
 (segment (start 111.102101 128.490601) (end 106.68 126.492) (width 0.25) (layer F.Cu) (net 6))
 (segment (start 112.5775 129.3406) (end 111.727501 128.490601) (width 0.25) (layer F.Cu) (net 6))
 (segment (start 111.727501 128.490601) (end 111.102101 128.490601) (width 0.25) (layer F.Cu) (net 6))
 (segment (start 106.68 124.868998) (end 106.68 126.492) (width 0.25) (layer F.Cu) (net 6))
 (segment (start 104.648 122.836998) (end 106.68 124.868998) (width 0.25) (layer F.Cu) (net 6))
 (segment (start 104.648 121.158) (end 104.648 122.836998) (width 0.25) (layer F.Cu) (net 6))
 (segment (start 109.259001 117.740799) (end 110.109 116.8908) (width 0.25) (layer F.Cu) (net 6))
 (segment (start 106.96681 120.03299) (end 109.259001 117.740799) (width 0.25) (layer F.Cu) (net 6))
 (segment (start 105.77301 120.03299) (end 106.96681 120.03299) (width 0.25) (layer F.Cu) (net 6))
 (segment (start 104.648 121.158) (end 105.77301 120.03299) (width 0.25) (layer F.Cu) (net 6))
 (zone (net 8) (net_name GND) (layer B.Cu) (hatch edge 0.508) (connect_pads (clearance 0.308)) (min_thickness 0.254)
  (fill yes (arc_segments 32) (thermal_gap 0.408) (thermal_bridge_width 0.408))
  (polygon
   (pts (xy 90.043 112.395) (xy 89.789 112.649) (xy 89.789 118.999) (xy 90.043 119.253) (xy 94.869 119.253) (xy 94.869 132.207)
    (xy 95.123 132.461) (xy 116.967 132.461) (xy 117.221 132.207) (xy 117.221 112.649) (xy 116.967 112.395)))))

